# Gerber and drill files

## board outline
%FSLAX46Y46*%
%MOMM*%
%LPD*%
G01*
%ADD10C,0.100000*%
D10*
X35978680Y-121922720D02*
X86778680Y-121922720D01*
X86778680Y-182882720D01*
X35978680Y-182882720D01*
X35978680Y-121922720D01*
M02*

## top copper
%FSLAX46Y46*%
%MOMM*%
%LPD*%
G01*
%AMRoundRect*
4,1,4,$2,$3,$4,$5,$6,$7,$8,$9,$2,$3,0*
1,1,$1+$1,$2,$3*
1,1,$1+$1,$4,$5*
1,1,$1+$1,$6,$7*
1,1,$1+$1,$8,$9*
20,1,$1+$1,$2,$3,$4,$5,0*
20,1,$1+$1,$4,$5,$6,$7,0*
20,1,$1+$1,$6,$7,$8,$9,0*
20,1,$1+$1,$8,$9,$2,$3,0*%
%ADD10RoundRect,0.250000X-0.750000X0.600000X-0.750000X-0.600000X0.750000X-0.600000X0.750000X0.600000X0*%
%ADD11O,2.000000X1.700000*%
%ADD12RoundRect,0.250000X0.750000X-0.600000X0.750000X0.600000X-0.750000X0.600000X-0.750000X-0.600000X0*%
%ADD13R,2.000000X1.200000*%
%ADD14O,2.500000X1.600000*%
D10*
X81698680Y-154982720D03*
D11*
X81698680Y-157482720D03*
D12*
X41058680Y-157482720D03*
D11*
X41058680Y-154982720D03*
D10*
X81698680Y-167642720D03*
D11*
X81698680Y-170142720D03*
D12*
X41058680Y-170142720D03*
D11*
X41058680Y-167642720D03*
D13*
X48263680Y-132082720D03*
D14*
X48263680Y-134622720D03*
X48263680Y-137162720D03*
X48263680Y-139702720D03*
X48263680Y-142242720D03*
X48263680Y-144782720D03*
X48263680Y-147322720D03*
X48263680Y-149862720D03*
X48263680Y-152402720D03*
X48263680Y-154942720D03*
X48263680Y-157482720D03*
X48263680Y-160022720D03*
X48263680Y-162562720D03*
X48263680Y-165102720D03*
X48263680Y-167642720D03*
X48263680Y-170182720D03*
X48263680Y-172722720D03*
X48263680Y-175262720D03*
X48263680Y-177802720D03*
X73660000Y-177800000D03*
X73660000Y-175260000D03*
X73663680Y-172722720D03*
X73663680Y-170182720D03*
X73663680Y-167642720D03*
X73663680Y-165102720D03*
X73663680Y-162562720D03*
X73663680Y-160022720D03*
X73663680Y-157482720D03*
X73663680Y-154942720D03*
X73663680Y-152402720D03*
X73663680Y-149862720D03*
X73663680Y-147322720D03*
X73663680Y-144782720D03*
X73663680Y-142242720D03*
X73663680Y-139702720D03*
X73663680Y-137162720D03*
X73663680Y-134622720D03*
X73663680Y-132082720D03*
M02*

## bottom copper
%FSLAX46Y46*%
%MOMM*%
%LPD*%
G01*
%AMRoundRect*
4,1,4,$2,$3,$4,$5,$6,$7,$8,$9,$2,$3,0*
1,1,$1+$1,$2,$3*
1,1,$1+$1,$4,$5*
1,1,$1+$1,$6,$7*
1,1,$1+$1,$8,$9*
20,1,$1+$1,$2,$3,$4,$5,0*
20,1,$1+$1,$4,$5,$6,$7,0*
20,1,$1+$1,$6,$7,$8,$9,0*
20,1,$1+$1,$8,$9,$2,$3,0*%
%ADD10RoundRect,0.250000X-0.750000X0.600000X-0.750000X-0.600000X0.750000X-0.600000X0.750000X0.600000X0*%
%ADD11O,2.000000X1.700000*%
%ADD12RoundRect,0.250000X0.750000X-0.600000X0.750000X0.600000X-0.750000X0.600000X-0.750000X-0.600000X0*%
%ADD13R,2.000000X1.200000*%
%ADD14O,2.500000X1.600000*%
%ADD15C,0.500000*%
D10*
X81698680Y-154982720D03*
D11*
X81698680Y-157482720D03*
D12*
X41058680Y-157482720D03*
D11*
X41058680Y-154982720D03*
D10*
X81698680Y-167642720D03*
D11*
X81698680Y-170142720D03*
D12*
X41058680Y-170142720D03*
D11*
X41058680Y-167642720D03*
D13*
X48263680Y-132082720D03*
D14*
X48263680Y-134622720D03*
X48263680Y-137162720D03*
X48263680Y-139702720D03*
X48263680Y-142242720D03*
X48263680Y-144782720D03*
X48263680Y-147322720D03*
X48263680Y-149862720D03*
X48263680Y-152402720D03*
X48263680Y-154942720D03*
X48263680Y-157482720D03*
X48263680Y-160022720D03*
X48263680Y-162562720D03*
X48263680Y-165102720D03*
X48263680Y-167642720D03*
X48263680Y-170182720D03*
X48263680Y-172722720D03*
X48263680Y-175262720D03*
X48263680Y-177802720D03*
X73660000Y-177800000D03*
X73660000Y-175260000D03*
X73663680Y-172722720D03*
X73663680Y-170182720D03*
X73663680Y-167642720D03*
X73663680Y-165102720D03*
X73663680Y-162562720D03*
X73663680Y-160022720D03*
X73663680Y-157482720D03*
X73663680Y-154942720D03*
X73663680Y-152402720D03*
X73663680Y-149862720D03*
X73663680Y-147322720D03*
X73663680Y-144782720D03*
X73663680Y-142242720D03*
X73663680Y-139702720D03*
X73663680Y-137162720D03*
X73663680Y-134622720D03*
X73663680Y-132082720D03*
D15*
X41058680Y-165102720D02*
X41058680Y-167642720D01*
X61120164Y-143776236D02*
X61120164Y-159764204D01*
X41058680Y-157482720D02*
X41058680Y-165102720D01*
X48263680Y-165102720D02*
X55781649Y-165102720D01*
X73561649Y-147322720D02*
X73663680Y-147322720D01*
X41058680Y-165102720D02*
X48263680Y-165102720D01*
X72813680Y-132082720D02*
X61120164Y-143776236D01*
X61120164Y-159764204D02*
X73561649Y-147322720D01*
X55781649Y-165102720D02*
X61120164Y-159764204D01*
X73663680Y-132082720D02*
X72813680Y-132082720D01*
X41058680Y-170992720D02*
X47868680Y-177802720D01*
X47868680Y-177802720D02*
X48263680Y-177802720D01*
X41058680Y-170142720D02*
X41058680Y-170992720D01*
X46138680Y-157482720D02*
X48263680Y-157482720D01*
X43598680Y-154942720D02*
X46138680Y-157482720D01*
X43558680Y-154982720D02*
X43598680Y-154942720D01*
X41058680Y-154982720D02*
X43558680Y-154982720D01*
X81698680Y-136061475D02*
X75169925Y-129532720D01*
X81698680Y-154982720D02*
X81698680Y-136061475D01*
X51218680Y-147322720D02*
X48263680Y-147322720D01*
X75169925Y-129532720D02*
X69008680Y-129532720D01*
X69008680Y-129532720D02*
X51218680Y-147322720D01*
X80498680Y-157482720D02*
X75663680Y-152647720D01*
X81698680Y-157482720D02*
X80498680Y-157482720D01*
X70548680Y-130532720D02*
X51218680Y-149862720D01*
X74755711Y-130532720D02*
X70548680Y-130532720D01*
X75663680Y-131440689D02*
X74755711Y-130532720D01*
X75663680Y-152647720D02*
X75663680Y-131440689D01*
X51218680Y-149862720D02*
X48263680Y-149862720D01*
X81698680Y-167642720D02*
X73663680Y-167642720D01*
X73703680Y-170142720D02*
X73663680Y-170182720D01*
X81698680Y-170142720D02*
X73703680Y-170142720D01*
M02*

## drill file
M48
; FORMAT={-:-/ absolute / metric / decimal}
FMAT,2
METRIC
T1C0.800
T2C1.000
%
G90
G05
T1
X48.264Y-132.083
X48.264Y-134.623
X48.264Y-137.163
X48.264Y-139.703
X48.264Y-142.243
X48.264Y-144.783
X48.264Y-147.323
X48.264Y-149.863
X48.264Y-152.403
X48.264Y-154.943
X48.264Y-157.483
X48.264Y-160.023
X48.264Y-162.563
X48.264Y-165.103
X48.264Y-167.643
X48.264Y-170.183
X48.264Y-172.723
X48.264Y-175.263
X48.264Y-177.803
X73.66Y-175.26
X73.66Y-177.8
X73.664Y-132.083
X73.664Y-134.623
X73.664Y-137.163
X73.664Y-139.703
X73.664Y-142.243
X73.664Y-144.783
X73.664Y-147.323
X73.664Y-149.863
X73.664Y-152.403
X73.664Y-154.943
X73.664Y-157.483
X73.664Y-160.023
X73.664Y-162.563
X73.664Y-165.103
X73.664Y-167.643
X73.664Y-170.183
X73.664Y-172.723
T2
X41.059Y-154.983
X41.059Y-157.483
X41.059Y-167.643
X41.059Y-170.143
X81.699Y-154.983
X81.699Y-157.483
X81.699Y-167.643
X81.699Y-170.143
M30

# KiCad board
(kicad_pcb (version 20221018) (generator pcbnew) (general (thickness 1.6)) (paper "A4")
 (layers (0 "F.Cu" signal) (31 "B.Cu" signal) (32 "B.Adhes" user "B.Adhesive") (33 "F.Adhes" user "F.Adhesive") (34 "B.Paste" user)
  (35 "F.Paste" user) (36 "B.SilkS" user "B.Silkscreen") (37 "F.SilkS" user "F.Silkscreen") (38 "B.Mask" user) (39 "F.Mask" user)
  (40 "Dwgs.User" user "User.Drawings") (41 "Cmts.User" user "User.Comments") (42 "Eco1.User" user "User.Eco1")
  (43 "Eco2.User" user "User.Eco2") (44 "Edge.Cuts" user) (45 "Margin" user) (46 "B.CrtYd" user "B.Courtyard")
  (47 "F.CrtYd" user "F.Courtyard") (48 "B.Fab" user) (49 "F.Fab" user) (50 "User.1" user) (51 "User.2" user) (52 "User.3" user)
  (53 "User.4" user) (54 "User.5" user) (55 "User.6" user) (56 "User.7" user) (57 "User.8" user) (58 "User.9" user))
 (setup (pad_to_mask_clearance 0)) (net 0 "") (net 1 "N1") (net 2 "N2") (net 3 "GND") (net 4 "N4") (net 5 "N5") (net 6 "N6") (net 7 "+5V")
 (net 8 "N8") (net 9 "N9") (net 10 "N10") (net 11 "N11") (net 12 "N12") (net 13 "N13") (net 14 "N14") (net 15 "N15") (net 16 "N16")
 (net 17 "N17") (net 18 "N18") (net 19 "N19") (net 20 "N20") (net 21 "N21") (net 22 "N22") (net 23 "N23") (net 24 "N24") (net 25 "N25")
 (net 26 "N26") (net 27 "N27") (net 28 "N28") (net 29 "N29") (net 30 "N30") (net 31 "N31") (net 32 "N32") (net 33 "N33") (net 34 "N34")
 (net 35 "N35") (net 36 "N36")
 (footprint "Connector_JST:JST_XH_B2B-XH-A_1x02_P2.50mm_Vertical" (layer "F.Cu") (at 81.69868 154.98272 -90)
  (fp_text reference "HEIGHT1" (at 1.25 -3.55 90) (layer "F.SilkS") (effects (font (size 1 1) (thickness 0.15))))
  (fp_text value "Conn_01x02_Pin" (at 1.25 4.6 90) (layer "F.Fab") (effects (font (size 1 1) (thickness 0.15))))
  (pad "1" thru_hole roundrect (at 0 0 270) (size 1.7 2) (drill 1) (layers "*.Cu" "*.Mask") (roundrect_rratio 0.1470588235) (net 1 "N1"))
  (pad "2" thru_hole oval (at 2.5 0 270) (size 1.7 2) (drill 1) (layers "*.Cu" "*.Mask") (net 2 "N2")))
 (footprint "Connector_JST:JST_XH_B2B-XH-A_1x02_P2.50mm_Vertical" (layer "F.Cu") (at 41.05868 157.48272 90)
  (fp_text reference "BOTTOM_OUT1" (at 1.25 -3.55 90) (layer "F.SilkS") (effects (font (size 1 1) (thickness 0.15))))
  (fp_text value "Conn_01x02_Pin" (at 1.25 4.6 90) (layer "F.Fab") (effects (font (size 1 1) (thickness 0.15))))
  (pad "1" thru_hole roundrect (at 0 0 90) (size 1.7 2) (drill 1) (layers "*.Cu" "*.Mask") (roundrect_rratio 0.1470588235) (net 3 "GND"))
  (pad "2" thru_hole oval (at 2.5 0 90) (size 1.7 2) (drill 1) (layers "*.Cu" "*.Mask") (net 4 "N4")))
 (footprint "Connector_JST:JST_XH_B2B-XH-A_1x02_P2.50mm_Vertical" (layer "F.Cu") (at 81.69868 167.64272 -90)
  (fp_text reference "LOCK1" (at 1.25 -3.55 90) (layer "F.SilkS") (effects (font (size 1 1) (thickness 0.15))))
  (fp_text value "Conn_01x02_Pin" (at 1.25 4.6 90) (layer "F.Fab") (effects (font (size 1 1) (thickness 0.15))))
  (pad "1" thru_hole roundrect (at 0 0 270) (size 1.7 2) (drill 1) (layers "*.Cu" "*.Mask") (roundrect_rratio 0.1470588235) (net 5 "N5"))
  (pad "2" thru_hole oval (at 2.5 0 270) (size 1.7 2) (drill 1) (layers "*.Cu" "*.Mask") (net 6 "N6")))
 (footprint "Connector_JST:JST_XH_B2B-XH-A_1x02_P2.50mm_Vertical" (layer "F.Cu") (at 41.05868 170.14272 90)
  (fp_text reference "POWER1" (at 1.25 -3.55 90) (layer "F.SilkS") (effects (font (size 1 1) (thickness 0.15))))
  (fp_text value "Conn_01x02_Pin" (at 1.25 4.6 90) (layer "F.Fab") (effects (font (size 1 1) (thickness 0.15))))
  (pad "1" thru_hole roundrect (at 0 0 90) (size 1.7 2) (drill 1) (layers "*.Cu" "*.Mask") (roundrect_rratio 0.1470588235) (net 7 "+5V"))
  (pad "2" thru_hole oval (at 2.5 0 90) (size 1.7 2) (drill 1) (layers "*.Cu" "*.Mask") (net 3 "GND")))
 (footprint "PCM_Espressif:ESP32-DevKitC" (layer "F.Cu") (at 48.26368 132.08272)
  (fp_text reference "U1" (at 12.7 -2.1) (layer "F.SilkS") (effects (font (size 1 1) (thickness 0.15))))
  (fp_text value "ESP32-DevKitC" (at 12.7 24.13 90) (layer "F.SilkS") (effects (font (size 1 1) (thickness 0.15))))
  (pad "1" thru_hole rect (at 0 0 270) (size 1.2 2) (drill 0.8) (layers "*.Cu" "*.Mask") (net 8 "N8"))
  (pad "2" thru_hole oval (at 0 2.54 270) (size 1.6 2.5) (drill 0.8) (layers "*.Cu" "*.Mask") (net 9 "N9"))
  (pad "3" thru_hole oval (at 0 5.08 270) (size 1.6 2.5) (drill 0.8) (layers "*.Cu" "*.Mask") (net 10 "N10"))
  (pad "4" thru_hole oval (at 0 7.62 270) (size 1.6 2.5) (drill 0.8) (layers "*.Cu" "*.Mask") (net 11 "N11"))
  (pad "5" thru_hole oval (at 0 10.16 270) (size 1.6 2.5) (drill 0.8) (layers "*.Cu" "*.Mask") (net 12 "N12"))
  (pad "6" thru_hole oval (at 0 12.7 270) (size 1.6 2.5) (drill 0.8) (layers "*.Cu" "*.Mask") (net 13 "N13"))
  (pad "7" thru_hole oval (at 0 15.24 270) (size 1.6 2.5) (drill 0.8) (layers "*.Cu" "*.Mask") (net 1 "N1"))
  (pad "8" thru_hole oval (at 0 17.78 270) (size 1.6 2.5) (drill 0.8) (layers "*.Cu" "*.Mask") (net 2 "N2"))
  (pad "9" thru_hole oval (at 0 20.32 270) (size 1.6 2.5) (drill 0.8) (layers "*.Cu" "*.Mask") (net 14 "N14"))
  (pad "10" thru_hole oval (at 0 22.86 270) (size 1.6 2.5) (drill 0.8) (layers "*.Cu" "*.Mask") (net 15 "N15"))
  (pad "11" thru_hole oval (at 0 25.4 270) (size 1.6 2.5) (drill 0.8) (layers "*.Cu" "*.Mask") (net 4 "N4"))
  (pad "12" thru_hole oval (at 0 27.94 270) (size 1.6 2.5) (drill 0.8) (layers "*.Cu" "*.Mask") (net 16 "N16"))
  (pad "13" thru_hole oval (at 0 30.48 270) (size 1.6 2.5) (drill 0.8) (layers "*.Cu" "*.Mask") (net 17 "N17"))
  (pad "14" thru_hole oval (at 0 33.02 270) (size 1.6 2.5) (drill 0.8) (layers "*.Cu" "*.Mask") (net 3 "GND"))
  (pad "15" thru_hole oval (at 0 35.56 270) (size 1.6 2.5) (drill 0.8) (layers "*.Cu" "*.Mask") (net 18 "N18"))
  (pad "16" thru_hole oval (at 0 38.1 270) (size 1.6 2.5) (drill 0.8) (layers "*.Cu" "*.Mask") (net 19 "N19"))
  (pad "17" thru_hole oval (at 0 40.64 270) (size 1.6 2.5) (drill 0.8) (layers "*.Cu" "*.Mask") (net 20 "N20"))
  (pad "18" thru_hole oval (at 0 43.18 270) (size 1.6 2.5) (drill 0.8) (layers "*.Cu" "*.Mask") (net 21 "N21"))
  (pad "19" thru_hole oval (at 0 45.72 270) (size 1.6 2.5) (drill 0.8) (layers "*.Cu" "*.Mask") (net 7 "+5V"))
  (pad "20" thru_hole oval (at 25.39632 45.71728 270) (size 1.6 2.5) (drill 0.8) (layers "*.Cu" "*.Mask") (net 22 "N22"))
  (pad "21" thru_hole oval (at 25.39632 43.17728 270) (size 1.6 2.5) (drill 0.8) (layers "*.Cu" "*.Mask") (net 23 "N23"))
  (pad "22" thru_hole oval (at 25.4 40.64 270) (size 1.6 2.5) (drill 0.8) (layers "*.Cu" "*.Mask") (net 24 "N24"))
  (pad "23" thru_hole oval (at 25.4 38.1 270) (size 1.6 2.5) (drill 0.8) (layers "*.Cu" "*.Mask") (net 6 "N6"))
  (pad "24" thru_hole oval (at 25.4 35.56 270) (size 1.6 2.5) (drill 0.8) (layers "*.Cu" "*.Mask") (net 5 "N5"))
  (pad "25" thru_hole oval (at 25.4 33.02 270) (size 1.6 2.5) (drill 0.8) (layers "*.Cu" "*.Mask") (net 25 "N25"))
  (pad "26" thru_hole oval (at 25.4 30.48 270) (size 1.6 2.5) (drill 0.8) (layers "*.Cu" "*.Mask") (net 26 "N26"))
  (pad "27" thru_hole oval (at 25.4 27.94 270) (size 1.6 2.5) (drill 0.8) (layers "*.Cu" "*.Mask") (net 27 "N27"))
  (pad "28" thru_hole oval (at 25.4 25.4 270) (size 1.6 2.5) (drill 0.8) (layers "*.Cu" "*.Mask") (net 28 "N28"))
  (pad "29" thru_hole oval (at 25.4 22.86 270) (size 1.6 2.5) (drill 0.8) (layers "*.Cu" "*.Mask") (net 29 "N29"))
  (pad "30" thru_hole oval (at 25.4 20.32 270) (size 1.6 2.5) (drill 0.8) (layers "*.Cu" "*.Mask") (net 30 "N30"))
  (pad "31" thru_hole oval (at 25.4 17.78 270) (size 1.6 2.5) (drill 0.8) (layers "*.Cu" "*.Mask") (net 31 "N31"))
  (pad "32" thru_hole oval (at 25.4 15.24 270) (size 1.6 2.5) (drill 0.8) (layers "*.Cu" "*.Mask") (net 3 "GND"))
  (pad "33" thru_hole oval (at 25.4 12.7 270) (size 1.6 2.5) (drill 0.8) (layers "*.Cu" "*.Mask") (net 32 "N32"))
  (pad "34" thru_hole oval (at 25.4 10.16 270) (size 1.6 2.5) (drill 0.8) (layers "*.Cu" "*.Mask") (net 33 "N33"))
  (pad "35" thru_hole oval (at 25.4 7.62 270) (size 1.6 2.5) (drill 0.8) (layers "*.Cu" "*.Mask") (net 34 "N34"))
  (pad "36" thru_hole oval (at 25.4 5.08 270) (size 1.6 2.5) (drill 0.8) (layers "*.Cu" "*.Mask") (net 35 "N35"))
  (pad "37" thru_hole oval (at 25.4 2.54 270) (size 1.6 2.5) (drill 0.8) (layers "*.Cu" "*.Mask") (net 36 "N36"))
  (pad "38" thru_hole oval (at 25.4 0 270) (size 1.6 2.5) (drill 0.8) (layers "*.Cu" "*.Mask") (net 3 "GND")))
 (gr_rect (start 35.97868 121.92272) (end 86.77868 182.88272) (stroke (width 0.1) (type default)) (fill none) (layer "Edge.Cuts"))
 (segment (start 41.05868 165.10272) (end 41.05868 167.64272) (width 0.5) (layer "B.Cu") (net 3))
 (segment (start 61.120164 143.776236) (end 61.120164 159.764204) (width 0.5) (layer "B.Cu") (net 3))
 (segment (start 41.05868 157.48272) (end 41.05868 165.10272) (width 0.5) (layer "B.Cu") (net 3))
 (segment (start 48.26368 165.10272) (end 55.781649 165.10272) (width 0.5) (layer "B.Cu") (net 3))
 (segment (start 73.561649 147.32272) (end 73.66368 147.32272) (width 0.5) (layer "B.Cu") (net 3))
 (segment (start 41.05868 165.10272) (end 48.26368 165.10272) (width 0.5) (layer "B.Cu") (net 3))
 (segment (start 72.81368 132.08272) (end 61.120164 143.776236) (width 0.5) (layer "B.Cu") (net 3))
 (segment (start 61.120164 159.764204) (end 73.561649 147.32272) (width 0.5) (layer "B.Cu") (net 3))
 (segment (start 55.781649 165.10272) (end 61.120164 159.764204) (width 0.5) (layer "B.Cu") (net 3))
 (segment (start 73.66368 132.08272) (end 72.81368 132.08272) (width 0.5) (layer "B.Cu") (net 3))
 (segment (start 41.05868 170.99272) (end 47.86868 177.80272) (width 0.5) (layer "B.Cu") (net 7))
 (segment (start 47.86868 177.80272) (end 48.26368 177.80272) (width 0.5) (layer "B.Cu") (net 7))
 (segment (start 41.05868 170.14272) (end 41.05868 170.99272) (width 0.5) (layer "B.Cu") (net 7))
 (segment (start 46.13868 157.48272) (end 48.26368 157.48272) (width 0.5) (layer "B.Cu") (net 4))
 (segment (start 43.59868 154.94272) (end 46.13868 157.48272) (width 0.5) (layer "B.Cu") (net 4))
 (segment (start 43.55868 154.98272) (end 43.59868 154.94272) (width 0.5) (layer "B.Cu") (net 4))
 (segment (start 41.05868 154.98272) (end 43.55868 154.98272) (width 0.5) (layer "B.Cu") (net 4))
 (segment (start 81.69868 136.061475) (end 75.169925 129.53272) (width 0.5) (layer "B.Cu") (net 1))
 (segment (start 81.69868 154.98272) (end 81.69868 136.061475) (width 0.5) (layer "B.Cu") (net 1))
 (segment (start 51.21868 147.32272) (end 48.26368 147.32272) (width 0.5) (layer "B.Cu") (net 1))
 (segment (start 75.169925 129.53272) (end 69.00868 129.53272) (width 0.5) (layer "B.Cu") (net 1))
 (segment (start 69.00868 129.53272) (end 51.21868 147.32272) (width 0.5) (layer "B.Cu") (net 1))
 (segment (start 80.49868 157.48272) (end 75.66368 152.64772) (width 0.5) (layer "B.Cu") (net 2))
 (segment (start 81.69868 157.48272) (end 80.49868 157.48272) (width 0.5) (layer "B.Cu") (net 2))
 (segment (start 70.54868 130.53272) (end 51.21868 149.86272) (width 0.5) (layer "B.Cu") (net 2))
 (segment (start 74.755711 130.53272) (end 70.54868 130.53272) (width 0.5) (layer "B.Cu") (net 2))
 (segment (start 75.66368 131.440689) (end 74.755711 130.53272) (width 0.5) (layer "B.Cu") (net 2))
 (segment (start 75.66368 152.64772) (end 75.66368 131.440689) (width 0.5) (layer "B.Cu") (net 2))
 (segment (start 51.21868 149.86272) (end 48.26368 149.86272) (width 0.5) (layer "B.Cu") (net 2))
 (segment (start 81.69868 167.64272) (end 73.66368 167.64272) (width 0.5) (layer "B.Cu") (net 5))
 (segment (start 73.70368 170.14272) (end 73.66368 170.18272) (width 0.5) (layer "B.Cu") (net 6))
 (segment (start 81.69868 170.14272) (end 73.70368 170.14272) (width 0.5) (layer "B.Cu") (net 6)))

